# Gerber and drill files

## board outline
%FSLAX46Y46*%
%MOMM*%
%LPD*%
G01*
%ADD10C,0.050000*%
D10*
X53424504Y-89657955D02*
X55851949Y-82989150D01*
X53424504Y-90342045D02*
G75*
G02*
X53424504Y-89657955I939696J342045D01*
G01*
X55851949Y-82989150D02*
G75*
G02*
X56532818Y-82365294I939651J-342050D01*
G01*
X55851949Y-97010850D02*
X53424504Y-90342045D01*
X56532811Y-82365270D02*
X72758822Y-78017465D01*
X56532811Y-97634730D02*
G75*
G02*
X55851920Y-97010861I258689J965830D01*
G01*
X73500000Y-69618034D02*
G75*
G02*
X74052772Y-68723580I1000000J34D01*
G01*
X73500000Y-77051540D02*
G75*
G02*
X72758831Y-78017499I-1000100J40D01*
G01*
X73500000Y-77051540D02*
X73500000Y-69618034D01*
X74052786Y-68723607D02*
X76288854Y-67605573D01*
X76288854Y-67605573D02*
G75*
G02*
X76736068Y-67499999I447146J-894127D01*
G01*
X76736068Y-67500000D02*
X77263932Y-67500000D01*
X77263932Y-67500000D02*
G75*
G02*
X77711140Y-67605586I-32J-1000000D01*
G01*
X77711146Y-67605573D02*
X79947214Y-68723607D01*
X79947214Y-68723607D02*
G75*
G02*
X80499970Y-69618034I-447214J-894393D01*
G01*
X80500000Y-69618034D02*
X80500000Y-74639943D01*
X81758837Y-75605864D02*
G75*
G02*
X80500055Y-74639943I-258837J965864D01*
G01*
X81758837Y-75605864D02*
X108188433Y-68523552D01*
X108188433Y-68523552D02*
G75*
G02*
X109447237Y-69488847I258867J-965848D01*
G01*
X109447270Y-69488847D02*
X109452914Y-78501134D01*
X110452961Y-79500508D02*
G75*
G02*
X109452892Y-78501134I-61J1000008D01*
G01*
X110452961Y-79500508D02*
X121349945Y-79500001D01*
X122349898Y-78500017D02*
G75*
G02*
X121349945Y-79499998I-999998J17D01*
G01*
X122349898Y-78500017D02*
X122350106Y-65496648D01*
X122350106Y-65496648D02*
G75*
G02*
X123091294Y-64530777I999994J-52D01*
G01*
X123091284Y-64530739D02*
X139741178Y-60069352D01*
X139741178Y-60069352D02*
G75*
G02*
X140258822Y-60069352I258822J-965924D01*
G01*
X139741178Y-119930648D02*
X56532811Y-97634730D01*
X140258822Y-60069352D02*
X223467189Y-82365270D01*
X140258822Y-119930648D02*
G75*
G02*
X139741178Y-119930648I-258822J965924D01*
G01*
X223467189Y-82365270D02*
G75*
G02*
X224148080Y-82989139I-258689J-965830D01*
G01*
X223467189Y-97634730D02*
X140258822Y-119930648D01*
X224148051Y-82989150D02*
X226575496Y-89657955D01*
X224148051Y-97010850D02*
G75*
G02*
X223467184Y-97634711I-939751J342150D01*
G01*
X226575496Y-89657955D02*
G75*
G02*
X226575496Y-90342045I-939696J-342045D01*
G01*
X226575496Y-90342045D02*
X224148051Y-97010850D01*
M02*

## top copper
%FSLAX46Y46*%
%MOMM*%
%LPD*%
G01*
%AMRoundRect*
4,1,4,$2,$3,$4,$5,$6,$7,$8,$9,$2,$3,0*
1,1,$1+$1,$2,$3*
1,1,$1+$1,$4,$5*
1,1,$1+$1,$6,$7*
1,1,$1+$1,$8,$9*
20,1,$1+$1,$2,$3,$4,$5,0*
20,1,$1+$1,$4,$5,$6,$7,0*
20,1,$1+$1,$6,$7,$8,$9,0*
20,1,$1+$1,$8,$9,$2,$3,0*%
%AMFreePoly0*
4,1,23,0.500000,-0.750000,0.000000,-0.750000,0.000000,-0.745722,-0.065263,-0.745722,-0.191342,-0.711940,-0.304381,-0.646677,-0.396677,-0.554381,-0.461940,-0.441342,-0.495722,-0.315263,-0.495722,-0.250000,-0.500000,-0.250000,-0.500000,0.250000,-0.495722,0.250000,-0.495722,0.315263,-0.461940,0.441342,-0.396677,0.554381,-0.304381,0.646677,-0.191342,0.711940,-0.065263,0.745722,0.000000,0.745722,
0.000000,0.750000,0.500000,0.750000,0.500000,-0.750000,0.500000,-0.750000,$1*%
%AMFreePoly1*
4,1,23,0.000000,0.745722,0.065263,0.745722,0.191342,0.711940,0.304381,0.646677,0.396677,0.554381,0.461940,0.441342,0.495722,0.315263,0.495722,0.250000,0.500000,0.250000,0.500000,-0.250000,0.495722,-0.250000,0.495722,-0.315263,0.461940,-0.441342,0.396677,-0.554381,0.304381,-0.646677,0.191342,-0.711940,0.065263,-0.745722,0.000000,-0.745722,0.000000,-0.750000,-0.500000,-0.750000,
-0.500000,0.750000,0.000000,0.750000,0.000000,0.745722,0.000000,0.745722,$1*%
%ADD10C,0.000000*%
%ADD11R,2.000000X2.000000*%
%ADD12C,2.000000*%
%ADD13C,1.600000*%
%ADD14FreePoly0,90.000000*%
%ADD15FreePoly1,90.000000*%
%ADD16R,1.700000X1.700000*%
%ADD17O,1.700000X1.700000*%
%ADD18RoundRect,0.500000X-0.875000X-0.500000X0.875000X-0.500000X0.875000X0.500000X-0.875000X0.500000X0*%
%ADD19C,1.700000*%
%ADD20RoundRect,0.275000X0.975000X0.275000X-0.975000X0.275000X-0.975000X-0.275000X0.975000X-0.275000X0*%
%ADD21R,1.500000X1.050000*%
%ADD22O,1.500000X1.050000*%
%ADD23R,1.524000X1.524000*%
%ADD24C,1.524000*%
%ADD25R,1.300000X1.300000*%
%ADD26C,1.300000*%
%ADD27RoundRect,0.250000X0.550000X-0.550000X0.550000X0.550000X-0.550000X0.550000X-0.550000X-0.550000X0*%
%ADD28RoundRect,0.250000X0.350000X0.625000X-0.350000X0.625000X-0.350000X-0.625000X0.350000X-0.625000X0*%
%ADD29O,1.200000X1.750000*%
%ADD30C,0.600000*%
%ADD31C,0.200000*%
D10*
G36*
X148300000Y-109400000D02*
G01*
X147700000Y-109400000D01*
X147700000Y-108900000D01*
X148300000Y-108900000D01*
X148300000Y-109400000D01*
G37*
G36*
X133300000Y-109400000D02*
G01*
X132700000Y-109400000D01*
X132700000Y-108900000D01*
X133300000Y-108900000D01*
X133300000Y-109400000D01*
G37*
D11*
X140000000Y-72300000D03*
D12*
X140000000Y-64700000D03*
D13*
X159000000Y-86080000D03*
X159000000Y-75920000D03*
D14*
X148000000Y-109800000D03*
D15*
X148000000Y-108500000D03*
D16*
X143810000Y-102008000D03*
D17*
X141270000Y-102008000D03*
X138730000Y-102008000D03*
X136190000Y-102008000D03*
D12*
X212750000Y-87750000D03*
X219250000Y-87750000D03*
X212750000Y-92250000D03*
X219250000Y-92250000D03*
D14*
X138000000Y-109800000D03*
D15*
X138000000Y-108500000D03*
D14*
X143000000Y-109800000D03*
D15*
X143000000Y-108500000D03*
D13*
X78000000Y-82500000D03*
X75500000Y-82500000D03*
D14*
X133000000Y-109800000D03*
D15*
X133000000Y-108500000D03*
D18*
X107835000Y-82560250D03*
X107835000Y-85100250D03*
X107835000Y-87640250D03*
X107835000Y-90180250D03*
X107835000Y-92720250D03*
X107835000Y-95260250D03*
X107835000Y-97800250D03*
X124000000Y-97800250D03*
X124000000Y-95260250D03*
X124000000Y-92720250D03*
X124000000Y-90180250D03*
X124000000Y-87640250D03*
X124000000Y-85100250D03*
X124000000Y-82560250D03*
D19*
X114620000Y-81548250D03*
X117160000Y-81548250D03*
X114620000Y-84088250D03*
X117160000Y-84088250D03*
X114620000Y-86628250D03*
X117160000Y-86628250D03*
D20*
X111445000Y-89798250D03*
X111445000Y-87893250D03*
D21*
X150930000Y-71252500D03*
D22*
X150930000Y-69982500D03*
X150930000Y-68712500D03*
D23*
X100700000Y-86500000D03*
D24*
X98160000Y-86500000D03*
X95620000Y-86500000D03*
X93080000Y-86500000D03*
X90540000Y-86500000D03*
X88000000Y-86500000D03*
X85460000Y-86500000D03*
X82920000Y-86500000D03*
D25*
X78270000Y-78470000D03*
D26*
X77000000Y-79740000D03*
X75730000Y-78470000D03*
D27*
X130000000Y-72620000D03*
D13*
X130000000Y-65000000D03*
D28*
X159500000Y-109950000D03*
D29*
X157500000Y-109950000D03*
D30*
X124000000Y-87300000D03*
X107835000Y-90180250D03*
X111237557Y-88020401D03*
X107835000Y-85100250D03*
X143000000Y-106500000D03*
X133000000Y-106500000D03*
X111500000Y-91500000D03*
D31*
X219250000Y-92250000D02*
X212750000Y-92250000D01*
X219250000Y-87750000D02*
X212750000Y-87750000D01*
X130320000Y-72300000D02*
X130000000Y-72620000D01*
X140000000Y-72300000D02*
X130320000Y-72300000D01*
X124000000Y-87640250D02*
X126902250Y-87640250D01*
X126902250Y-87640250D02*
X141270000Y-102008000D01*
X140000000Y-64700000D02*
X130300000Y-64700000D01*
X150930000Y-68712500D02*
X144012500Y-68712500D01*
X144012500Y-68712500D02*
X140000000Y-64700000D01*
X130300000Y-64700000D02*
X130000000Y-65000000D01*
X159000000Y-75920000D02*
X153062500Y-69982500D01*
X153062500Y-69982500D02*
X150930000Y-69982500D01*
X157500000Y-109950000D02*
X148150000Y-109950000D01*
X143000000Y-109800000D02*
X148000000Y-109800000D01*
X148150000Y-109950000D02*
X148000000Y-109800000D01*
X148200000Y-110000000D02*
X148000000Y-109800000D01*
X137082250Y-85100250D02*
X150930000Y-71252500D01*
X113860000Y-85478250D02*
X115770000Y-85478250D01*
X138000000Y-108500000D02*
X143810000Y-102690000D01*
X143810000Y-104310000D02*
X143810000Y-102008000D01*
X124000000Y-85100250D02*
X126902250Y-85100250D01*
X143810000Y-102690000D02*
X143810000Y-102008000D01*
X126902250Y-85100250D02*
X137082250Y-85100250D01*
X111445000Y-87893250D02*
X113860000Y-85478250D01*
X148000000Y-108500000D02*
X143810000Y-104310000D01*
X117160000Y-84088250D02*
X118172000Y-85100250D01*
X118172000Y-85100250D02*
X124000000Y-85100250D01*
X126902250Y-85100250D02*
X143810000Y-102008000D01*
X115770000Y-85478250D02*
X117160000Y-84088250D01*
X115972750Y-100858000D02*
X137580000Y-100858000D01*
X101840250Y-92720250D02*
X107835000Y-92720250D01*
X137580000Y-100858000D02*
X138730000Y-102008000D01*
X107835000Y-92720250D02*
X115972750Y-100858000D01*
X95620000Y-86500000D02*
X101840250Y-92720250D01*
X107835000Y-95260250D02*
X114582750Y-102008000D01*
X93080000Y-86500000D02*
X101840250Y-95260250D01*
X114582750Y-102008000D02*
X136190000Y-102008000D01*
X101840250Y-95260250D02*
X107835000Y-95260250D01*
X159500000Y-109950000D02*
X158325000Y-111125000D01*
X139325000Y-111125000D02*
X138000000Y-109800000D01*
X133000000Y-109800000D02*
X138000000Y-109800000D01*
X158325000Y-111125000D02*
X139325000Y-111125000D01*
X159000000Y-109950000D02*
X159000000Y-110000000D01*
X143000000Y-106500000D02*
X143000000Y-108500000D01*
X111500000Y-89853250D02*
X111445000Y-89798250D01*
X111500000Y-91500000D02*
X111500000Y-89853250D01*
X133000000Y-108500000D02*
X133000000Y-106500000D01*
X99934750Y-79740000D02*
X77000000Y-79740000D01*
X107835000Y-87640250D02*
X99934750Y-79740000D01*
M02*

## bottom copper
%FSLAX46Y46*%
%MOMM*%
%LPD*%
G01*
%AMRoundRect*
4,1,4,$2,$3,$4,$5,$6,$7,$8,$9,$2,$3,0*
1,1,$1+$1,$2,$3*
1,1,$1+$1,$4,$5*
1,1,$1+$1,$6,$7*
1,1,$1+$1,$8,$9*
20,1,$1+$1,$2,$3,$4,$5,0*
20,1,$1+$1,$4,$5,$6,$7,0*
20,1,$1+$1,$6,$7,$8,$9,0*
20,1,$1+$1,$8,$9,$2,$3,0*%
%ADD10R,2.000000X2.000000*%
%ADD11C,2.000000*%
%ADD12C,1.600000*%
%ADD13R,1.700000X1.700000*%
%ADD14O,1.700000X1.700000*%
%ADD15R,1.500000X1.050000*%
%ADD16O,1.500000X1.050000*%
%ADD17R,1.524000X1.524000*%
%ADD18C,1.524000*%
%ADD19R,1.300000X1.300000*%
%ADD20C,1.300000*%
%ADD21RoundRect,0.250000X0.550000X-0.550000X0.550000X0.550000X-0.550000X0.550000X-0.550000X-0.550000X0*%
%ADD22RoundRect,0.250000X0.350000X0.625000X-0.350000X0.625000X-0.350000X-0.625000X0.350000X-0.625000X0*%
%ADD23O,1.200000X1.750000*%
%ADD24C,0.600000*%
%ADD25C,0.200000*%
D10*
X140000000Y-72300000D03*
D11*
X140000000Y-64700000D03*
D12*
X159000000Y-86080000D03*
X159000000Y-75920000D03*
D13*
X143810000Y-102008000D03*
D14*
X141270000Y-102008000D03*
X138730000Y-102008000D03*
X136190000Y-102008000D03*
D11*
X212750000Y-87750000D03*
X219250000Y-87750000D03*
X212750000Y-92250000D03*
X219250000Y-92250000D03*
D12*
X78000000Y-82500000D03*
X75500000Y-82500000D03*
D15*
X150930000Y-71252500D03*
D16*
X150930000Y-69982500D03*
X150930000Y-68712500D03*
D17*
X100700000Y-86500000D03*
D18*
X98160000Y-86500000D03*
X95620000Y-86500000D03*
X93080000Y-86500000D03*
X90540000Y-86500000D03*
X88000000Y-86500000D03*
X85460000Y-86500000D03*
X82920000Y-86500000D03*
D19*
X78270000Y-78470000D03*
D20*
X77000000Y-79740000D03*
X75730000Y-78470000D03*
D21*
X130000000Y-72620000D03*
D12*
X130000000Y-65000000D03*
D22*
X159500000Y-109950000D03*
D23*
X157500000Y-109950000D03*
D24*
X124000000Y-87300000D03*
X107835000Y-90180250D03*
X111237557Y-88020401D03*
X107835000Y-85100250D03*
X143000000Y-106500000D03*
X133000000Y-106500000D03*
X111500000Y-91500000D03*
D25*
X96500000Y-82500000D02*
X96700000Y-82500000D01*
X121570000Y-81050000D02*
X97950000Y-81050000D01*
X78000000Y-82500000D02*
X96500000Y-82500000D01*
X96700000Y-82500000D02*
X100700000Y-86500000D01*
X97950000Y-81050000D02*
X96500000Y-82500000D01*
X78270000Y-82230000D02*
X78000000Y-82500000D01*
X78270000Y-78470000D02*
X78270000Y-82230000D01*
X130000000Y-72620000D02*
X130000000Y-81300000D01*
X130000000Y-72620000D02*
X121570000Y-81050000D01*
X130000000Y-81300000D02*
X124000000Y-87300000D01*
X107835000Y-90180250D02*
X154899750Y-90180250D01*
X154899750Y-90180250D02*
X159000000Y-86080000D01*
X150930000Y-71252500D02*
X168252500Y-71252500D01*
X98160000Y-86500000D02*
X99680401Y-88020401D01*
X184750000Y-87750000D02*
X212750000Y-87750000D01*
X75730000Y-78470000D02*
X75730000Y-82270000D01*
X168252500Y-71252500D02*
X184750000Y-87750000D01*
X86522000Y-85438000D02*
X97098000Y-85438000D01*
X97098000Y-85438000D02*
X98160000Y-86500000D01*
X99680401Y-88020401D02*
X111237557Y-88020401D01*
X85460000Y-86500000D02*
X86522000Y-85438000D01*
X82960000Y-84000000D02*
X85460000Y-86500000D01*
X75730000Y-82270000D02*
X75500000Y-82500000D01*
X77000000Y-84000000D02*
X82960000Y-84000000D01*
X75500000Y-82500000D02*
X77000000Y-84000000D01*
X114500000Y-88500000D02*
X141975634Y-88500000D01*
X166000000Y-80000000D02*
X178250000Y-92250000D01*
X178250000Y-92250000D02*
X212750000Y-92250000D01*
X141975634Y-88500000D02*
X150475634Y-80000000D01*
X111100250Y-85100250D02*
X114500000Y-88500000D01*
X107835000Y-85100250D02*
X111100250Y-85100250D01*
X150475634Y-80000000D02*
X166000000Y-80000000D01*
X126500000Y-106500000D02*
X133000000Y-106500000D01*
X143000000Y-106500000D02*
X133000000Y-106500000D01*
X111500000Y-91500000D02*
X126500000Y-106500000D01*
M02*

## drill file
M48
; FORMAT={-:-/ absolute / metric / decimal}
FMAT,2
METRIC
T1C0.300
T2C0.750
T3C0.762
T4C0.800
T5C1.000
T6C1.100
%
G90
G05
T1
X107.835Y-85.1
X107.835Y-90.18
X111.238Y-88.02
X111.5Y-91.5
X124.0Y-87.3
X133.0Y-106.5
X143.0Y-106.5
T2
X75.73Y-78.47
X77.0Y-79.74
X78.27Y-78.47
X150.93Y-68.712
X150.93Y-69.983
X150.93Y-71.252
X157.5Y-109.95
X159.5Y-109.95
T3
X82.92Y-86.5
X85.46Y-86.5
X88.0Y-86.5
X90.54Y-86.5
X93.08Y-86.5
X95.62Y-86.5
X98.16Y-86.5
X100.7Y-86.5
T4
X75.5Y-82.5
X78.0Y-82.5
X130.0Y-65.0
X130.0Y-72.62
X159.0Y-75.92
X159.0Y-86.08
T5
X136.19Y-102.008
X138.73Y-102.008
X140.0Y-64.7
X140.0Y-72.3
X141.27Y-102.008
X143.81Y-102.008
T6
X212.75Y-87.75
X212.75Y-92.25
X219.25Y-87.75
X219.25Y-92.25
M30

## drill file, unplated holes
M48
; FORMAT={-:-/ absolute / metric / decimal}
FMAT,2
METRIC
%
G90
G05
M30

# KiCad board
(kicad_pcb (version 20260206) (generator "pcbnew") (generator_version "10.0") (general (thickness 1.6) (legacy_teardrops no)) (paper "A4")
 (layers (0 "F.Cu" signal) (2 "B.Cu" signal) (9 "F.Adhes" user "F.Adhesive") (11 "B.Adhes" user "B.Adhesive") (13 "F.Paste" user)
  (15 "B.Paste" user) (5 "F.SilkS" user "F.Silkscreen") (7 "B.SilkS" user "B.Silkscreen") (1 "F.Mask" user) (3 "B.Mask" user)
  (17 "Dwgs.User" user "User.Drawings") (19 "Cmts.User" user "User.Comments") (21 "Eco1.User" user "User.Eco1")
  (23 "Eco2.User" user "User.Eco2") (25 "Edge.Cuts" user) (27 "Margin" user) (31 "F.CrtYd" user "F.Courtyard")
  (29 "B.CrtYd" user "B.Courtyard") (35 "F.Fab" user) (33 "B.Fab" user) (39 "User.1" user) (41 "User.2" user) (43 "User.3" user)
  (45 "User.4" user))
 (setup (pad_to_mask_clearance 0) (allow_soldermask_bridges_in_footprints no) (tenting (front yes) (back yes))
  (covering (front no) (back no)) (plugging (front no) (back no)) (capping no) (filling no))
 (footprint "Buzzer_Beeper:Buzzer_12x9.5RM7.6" (layer "F.Cu") (at 140 72.3 90)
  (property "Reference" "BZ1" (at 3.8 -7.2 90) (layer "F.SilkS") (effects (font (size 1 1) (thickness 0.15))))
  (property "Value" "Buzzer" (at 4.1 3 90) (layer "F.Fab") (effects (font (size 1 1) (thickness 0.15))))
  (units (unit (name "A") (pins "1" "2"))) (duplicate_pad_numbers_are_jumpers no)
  (pad "1" thru_hole rect (at 0 0 90) (size 2 2) (drill 1) (layers "*.Cu" "*.Mask") (remove_unused_layers no) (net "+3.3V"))
  (pad "2" thru_hole circle (at 7.6 0 90) (size 2 2) (drill 1) (layers "*.Cu" "*.Mask") (remove_unused_layers no) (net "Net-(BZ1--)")))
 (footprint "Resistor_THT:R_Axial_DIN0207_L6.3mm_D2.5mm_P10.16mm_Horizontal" (layer "F.Cu") (at 159 86.08 90)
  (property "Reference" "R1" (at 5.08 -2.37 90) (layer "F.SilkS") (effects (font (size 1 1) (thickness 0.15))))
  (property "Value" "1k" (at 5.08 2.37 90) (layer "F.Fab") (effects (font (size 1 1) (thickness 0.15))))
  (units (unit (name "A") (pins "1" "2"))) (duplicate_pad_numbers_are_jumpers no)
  (pad "1" thru_hole circle (at 0 0 90) (size 1.6 1.6) (drill 0.8) (layers "*.Cu" "*.Mask") (remove_unused_layers no)
   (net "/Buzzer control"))
  (pad "2" thru_hole circle (at 10.16 0 90) (size 1.6 1.6) (drill 0.8) (layers "*.Cu" "*.Mask") (remove_unused_layers no) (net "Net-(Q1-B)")))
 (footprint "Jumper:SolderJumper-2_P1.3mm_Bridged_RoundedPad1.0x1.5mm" (layer "F.Cu") (at 148 109.15 90)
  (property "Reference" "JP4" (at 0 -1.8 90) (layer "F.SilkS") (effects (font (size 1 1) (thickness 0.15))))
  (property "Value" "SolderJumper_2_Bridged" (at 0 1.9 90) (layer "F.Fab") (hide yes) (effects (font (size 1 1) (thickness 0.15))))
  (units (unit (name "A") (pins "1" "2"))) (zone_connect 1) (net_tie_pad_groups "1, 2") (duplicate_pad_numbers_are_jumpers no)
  (fp_poly (pts (xy 0.25 -0.3) (xy -0.25 -0.3) (xy -0.25 0.3) (xy 0.25 0.3)) (stroke (width 0) (type solid)) (fill yes) (layer "F.Cu"))
  (pad "1" smd custom (at -0.65 0 90) (size 1 0.5) (layers "F.Cu" "F.Mask") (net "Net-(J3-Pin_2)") (zone_connect 2)
   (thermal_bridge_angle 45) (options (clearance outline) (anchor rect)) (primitives))
  (pad "2" smd custom (at 0.65 0 90) (size 1 0.5) (layers "F.Cu" "F.Mask") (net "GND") (zone_connect 2) (thermal_bridge_angle 45)
   (options (clearance outline) (anchor rect)) (primitives)))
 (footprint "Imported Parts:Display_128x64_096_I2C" (layer "F.Cu") (at 140 102.008 180)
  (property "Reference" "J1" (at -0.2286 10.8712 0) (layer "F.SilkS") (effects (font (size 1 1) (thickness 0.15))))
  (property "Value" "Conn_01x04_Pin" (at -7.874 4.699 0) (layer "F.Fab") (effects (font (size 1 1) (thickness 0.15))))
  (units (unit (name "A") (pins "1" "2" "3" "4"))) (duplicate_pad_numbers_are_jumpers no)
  (pad "1" thru_hole rect (at -3.81 0 270) (size 1.7 1.7) (drill 1) (layers "*.Cu" "*.Mask") (remove_unused_layers no) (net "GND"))
  (pad "2" thru_hole oval (at -1.27 0 270) (size 1.7 1.7) (drill 1) (layers "*.Cu" "*.Mask") (remove_unused_layers no) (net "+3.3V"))
  (pad "3" thru_hole oval (at 1.27 0 270) (size 1.7 1.7) (drill 1) (layers "*.Cu" "*.Mask") (remove_unused_layers no) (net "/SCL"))
  (pad "4" thru_hole oval (at 3.81 0 270) (size 1.7 1.7) (drill 1) (layers "*.Cu" "*.Mask") (remove_unused_layers no) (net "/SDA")))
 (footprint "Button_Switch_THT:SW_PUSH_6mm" (layer "F.Cu") (at 212.75 87.75)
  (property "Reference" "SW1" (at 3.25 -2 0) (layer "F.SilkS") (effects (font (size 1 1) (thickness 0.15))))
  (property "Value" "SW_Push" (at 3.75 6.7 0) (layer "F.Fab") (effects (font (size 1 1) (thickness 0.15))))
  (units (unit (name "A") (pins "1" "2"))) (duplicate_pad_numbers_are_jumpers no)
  (pad "1" thru_hole circle (at 0 0 90) (size 2 2) (drill 1.1) (layers "*.Cu" "*.Mask") (remove_unused_layers no) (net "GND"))
  (pad "1" thru_hole circle (at 6.5 0 90) (size 2 2) (drill 1.1) (layers "*.Cu" "*.Mask") (remove_unused_layers no) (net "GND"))
  (pad "2" thru_hole circle (at 0 4.5 90) (size 2 2) (drill 1.1) (layers "*.Cu" "*.Mask") (remove_unused_layers no) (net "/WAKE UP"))
  (pad "2" thru_hole circle (at 6.5 4.5 90) (size 2 2) (drill 1.1) (layers "*.Cu" "*.Mask") (remove_unused_layers no) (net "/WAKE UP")))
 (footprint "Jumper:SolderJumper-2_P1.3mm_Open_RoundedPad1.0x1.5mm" (layer "F.Cu") (at 138 109.15 90)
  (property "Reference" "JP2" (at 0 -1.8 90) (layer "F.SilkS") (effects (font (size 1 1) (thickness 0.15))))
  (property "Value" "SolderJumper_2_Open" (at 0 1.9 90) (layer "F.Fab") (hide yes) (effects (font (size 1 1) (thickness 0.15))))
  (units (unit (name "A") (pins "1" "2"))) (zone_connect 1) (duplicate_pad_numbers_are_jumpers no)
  (pad "1" smd custom (at -0.65 0 90) (size 1 0.5) (layers "F.Cu" "F.Mask") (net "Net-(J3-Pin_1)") (zone_connect 2)
   (thermal_bridge_angle 45) (options (clearance outline) (anchor rect)) (primitives))
  (pad "2" smd custom (at 0.65 0 90) (size 1 0.5) (layers "F.Cu" "F.Mask") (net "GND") (zone_connect 2) (thermal_bridge_angle 45)
   (options (clearance outline) (anchor rect)) (primitives)))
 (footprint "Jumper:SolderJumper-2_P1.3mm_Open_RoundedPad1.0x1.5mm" (layer "F.Cu") (at 143 109.15 90)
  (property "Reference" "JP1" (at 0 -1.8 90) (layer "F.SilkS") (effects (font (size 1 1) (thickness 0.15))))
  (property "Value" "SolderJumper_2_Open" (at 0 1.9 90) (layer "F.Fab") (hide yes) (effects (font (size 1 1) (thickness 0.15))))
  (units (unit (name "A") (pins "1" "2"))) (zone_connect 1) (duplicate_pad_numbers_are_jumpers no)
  (pad "1" smd custom (at -0.65 0 90) (size 1 0.5) (layers "F.Cu" "F.Mask") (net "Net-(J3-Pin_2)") (zone_connect 2)
   (thermal_bridge_angle 45) (options (clearance outline) (anchor rect)) (primitives))
  (pad "2" smd custom (at 0.65 0 90) (size 1 0.5) (layers "F.Cu" "F.Mask") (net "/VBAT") (zone_connect 2) (thermal_bridge_angle 45)
   (options (clearance outline) (anchor rect)) (primitives)))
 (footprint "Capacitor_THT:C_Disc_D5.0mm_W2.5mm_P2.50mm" (layer "F.Cu") (at 78 82.5 180)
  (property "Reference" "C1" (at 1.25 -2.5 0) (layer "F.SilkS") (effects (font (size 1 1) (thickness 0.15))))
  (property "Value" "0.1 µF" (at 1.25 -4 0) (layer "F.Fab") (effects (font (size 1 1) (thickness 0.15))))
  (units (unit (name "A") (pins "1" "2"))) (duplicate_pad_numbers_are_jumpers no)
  (pad "1" thru_hole circle (at 0 0 180) (size 1.6 1.6) (drill 0.8) (layers "*.Cu" "*.Mask") (remove_unused_layers no) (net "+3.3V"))
  (pad "2" thru_hole circle (at 2.5 0 180) (size 1.6 1.6) (drill 0.8) (layers "*.Cu" "*.Mask") (remove_unused_layers no) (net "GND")))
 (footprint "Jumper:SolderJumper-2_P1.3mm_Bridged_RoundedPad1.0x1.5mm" (layer "F.Cu") (at 133 109.15 90)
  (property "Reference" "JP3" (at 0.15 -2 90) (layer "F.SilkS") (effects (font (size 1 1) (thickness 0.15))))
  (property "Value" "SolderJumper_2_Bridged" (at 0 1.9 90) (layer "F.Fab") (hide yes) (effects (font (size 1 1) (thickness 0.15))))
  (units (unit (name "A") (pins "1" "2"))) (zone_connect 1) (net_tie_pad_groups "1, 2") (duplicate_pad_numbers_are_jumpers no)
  (fp_poly (pts (xy 0.25 -0.3) (xy -0.25 -0.3) (xy -0.25 0.3) (xy 0.25 0.3)) (stroke (width 0) (type solid)) (fill yes) (layer "F.Cu"))
  (pad "1" smd custom (at -0.65 0 90) (size 1 0.5) (layers "F.Cu" "F.Mask") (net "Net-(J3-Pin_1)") (zone_connect 2)
   (thermal_bridge_angle 45) (options (clearance outline) (anchor rect)) (primitives))
  (pad "2" smd custom (at 0.65 0 90) (size 1 0.5) (layers "F.Cu" "F.Mask") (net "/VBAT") (zone_connect 2) (thermal_bridge_angle 45)
   (options (clearance outline) (anchor rect)) (primitives)))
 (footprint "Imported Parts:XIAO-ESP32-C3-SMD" (layer "F.Cu") (at 107 100.68025)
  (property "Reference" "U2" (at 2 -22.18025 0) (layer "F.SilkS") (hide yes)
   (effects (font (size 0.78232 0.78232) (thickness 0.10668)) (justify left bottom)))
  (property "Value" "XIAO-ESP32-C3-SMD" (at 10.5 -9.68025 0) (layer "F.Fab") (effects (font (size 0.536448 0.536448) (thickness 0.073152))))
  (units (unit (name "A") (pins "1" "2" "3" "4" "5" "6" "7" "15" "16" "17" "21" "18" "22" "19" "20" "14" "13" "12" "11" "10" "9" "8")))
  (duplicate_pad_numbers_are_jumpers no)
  (pad "1" smd roundrect (at 0.835 -18.12) (size 2.75 2) (layers "F.Cu" "F.Mask" "F.Paste") (roundrect_rratio 0.25)
   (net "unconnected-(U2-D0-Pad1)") (solder_mask_margin 0.0508) (thermal_bridge_angle 45))
  (pad "2" smd roundrect (at 0.835 -15.58) (size 2.75 2) (layers "F.Cu" "F.Mask" "F.Paste") (roundrect_rratio 0.25) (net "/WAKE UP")
   (solder_mask_margin 0.0508) (thermal_bridge_angle 45))
  (pad "3" smd roundrect (at 0.835 -13.04) (size 2.75 2) (layers "F.Cu" "F.Mask" "F.Paste") (roundrect_rratio 0.25) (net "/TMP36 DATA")
   (solder_mask_margin 0.0508) (thermal_bridge_angle 45))
  (pad "4" smd roundrect (at 0.835 -10.5) (size 2.75 2) (layers "F.Cu" "F.Mask" "F.Paste") (roundrect_rratio 0.25) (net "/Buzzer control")
   (solder_mask_margin 0.0508) (thermal_bridge_angle 45))
  (pad "5" smd roundrect (at 0.835 -7.96) (size 2.75 2) (layers "F.Cu" "F.Mask" "F.Paste") (roundrect_rratio 0.25) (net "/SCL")
   (solder_mask_margin 0.0508) (thermal_bridge_angle 45))
  (pad "6" smd roundrect (at 0.835 -5.42) (size 2.75 2) (layers "F.Cu" "F.Mask" "F.Paste") (roundrect_rratio 0.25) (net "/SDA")
   (solder_mask_margin 0.0508) (thermal_bridge_angle 45))
  (pad "7" smd roundrect (at 0.835 -2.88) (size 2.75 2) (layers "F.Cu" "F.Mask" "F.Paste") (roundrect_rratio 0.25)
   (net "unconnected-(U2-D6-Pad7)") (solder_mask_margin 0.0508) (thermal_bridge_angle 45))
  (pad "8" smd roundrect (at 17 -2.88) (size 2.75 2) (layers "F.Cu" "F.Mask" "F.Paste") (roundrect_rratio 0.25)
   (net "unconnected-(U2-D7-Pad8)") (solder_mask_margin 0.0508) (thermal_bridge_angle 45))
  (pad "9" smd roundrect (at 17 -5.42) (size 2.75 2) (layers "F.Cu" "F.Mask" "F.Paste") (roundrect_rratio 0.25)
   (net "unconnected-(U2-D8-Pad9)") (solder_mask_margin 0.0508) (thermal_bridge_angle 45))
  (pad "10" smd roundrect (at 17 -7.96) (size 2.75 2) (layers "F.Cu" "F.Mask" "F.Paste") (roundrect_rratio 0.25)
   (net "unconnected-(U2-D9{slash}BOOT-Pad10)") (solder_mask_margin 0.0508) (thermal_bridge_angle 45))
  (pad "11" smd roundrect (at 17 -10.5) (size 2.75 2) (layers "F.Cu" "F.Mask" "F.Paste") (roundrect_rratio 0.25)
   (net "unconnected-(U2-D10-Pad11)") (solder_mask_margin 0.0508) (thermal_bridge_angle 45))
  (pad "12" smd roundrect (at 17 -13.04) (size 2.75 2) (layers "F.Cu" "F.Mask" "F.Paste") (roundrect_rratio 0.25) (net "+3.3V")
   (solder_mask_margin 0.0508) (thermal_bridge_angle 45))
  (pad "13" smd roundrect (at 17 -15.58) (size 2.75 2) (layers "F.Cu" "F.Mask" "F.Paste") (roundrect_rratio 0.25) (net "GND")
   (solder_mask_margin 0.0508) (thermal_bridge_angle 45))
  (pad "14" smd roundrect (at 17 -18.12) (size 2.75 2) (layers "F.Cu" "F.Mask" "F.Paste") (roundrect_rratio 0.25) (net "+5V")
   (solder_mask_margin 0.0508) (thermal_bridge_angle 45))
  (pad "15" smd circle (at 7.62 -19.132) (size 1.7 1.7) (layers "F.Cu" "F.Mask" "F.Paste") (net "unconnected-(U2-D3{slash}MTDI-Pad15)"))
  (pad "16" smd circle (at 10.16 -19.132) (size 1.7 1.7) (layers "F.Cu" "F.Mask" "F.Paste") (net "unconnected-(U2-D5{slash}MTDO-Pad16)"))
  (pad "17" smd circle (at 7.62 -16.592) (size 1.7 1.7) (layers "F.Cu" "F.Mask" "F.Paste") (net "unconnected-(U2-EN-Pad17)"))
  (pad "18" smd circle (at 10.16 -16.592) (size 1.7 1.7) (layers "F.Cu" "F.Mask" "F.Paste") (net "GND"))
  (pad "19" smd circle (at 7.62 -14.052) (size 1.7 1.7) (layers "F.Cu" "F.Mask" "F.Paste") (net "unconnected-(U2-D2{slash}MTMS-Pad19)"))
  (pad "20" smd circle (at 10.16 -14.052) (size 1.7 1.7) (layers "F.Cu" "F.Mask" "F.Paste") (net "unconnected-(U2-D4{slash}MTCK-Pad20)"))
  (pad "21" smd roundrect (at 4.445 -10.882 180) (size 2.5 1.1) (layers "F.Cu" "F.Mask" "F.Paste") (roundrect_rratio 0.25) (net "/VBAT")
   (thermal_bridge_angle 45))
  (pad "22" smd roundrect (at 4.445 -12.787 180) (size 2.5 1.1) (layers "F.Cu" "F.Mask" "F.Paste") (roundrect_rratio 0.25) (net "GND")
   (thermal_bridge_angle 45)))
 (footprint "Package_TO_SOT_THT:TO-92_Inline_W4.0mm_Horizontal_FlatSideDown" (layer "F.Cu") (at 150.93 71.2525 90)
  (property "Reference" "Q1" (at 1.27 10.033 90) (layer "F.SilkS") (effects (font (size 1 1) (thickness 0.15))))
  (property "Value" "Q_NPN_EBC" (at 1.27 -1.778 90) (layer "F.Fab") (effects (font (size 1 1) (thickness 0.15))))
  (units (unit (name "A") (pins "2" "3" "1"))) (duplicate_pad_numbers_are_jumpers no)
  (pad "1" thru_hole rect (at 0 0 90) (size 1.05 1.5) (drill 0.75) (layers "*.Cu" "*.Mask") (remove_unused_layers no) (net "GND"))
  (pad "2" thru_hole oval (at 1.27 0 90) (size 1.05 1.5) (drill 0.75) (layers "*.Cu" "*.Mask") (remove_unused_layers no) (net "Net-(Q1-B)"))
  (pad "3" thru_hole oval (at 2.54 0 90) (size 1.05 1.5) (drill 0.75) (layers "*.Cu" "*.Mask") (remove_unused_layers no) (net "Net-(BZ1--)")))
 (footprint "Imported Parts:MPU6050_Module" (layer "F.Cu") (at 100.7 86.5 -90)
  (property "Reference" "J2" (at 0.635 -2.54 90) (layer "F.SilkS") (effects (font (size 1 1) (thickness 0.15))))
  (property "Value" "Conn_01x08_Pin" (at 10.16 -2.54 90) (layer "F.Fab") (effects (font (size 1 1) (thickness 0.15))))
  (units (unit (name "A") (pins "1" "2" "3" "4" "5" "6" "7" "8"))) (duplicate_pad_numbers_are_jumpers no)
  (pad "1" thru_hole rect (at 0 0 270) (size 1.524 1.524) (drill 0.762) (layers "*.Cu" "*.Mask") (remove_unused_layers no) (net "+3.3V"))
  (pad "2" thru_hole circle (at 0 2.54 270) (size 1.524 1.524) (drill 0.762) (layers "*.Cu" "*.Mask") (remove_unused_layers no) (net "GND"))
  (pad "3" thru_hole circle (at 0 5.08 270) (size 1.524 1.524) (drill 0.762) (layers "*.Cu" "*.Mask") (remove_unused_layers no) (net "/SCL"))
  (pad "4" thru_hole circle (at 0 7.62 270) (size 1.524 1.524) (drill 0.762) (layers "*.Cu" "*.Mask") (remove_unused_layers no) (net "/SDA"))
  (pad "5" thru_hole circle (at 0 10.16 270) (size 1.524 1.524) (drill 0.762) (layers "*.Cu" "*.Mask") (remove_unused_layers no)
   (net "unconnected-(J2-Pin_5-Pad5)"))
  (pad "6" thru_hole circle (at 0 12.7 270) (size 1.524 1.524) (drill 0.762) (layers "*.Cu" "*.Mask") (remove_unused_layers no)
   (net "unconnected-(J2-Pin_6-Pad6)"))
  (pad "7" thru_hole circle (at 0 15.24 270) (size 1.524 1.524) (drill 0.762) (layers "*.Cu" "*.Mask") (remove_unused_layers no) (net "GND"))
  (pad "8" thru_hole circle (at 0 17.78 270) (size 1.524 1.524) (drill 0.762) (layers "*.Cu" "*.Mask") (remove_unused_layers no)
   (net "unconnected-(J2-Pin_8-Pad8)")))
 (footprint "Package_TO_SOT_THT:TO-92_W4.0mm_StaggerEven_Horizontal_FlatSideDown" (layer "F.Cu") (at 78.27 78.47 180)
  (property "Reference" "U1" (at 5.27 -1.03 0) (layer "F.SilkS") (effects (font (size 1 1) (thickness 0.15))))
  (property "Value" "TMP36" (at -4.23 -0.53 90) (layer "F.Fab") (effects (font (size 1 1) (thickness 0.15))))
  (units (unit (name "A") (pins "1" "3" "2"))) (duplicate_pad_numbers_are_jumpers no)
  (pad "1" thru_hole rect (at 0 0 270) (size 1.3 1.3) (drill 0.75) (layers "*.Cu" "*.Mask") (remove_unused_layers no) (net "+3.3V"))
  (pad "2" thru_hole circle (at 1.27 -1.27 270) (size 1.3 1.3) (drill 0.75) (layers "*.Cu" "*.Mask") (remove_unused_layers no)
   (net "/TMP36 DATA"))
  (pad "3" thru_hole circle (at 2.54 0 270) (size 1.3 1.3) (drill 0.75) (layers "*.Cu" "*.Mask") (remove_unused_layers no) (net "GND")))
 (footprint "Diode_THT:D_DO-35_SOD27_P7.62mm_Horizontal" (layer "F.Cu") (at 130 72.62 90)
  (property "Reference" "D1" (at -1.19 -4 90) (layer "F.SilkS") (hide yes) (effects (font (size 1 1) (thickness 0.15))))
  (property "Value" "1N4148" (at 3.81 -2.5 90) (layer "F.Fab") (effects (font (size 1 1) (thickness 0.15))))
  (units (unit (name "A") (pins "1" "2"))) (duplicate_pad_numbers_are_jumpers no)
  (pad "1" thru_hole roundrect (at 0 0 90) (size 1.6 1.6) (drill 0.8) (layers "*.Cu" "*.Mask") (remove_unused_layers no)
   (roundrect_rratio 0.15625) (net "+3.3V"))
  (pad "2" thru_hole circle (at 7.62 0 90) (size 1.6 1.6) (drill 0.8) (layers "*.Cu" "*.Mask") (remove_unused_layers no) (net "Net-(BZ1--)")))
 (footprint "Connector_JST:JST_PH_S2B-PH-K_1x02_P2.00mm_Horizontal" (layer "F.Cu") (at 159.5 109.95 180)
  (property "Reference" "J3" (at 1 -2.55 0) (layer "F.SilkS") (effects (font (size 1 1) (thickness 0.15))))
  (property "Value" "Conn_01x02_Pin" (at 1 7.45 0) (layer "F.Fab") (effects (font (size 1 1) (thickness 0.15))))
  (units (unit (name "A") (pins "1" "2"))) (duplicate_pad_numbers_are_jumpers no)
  (pad "1" thru_hole roundrect (at 0 0 180) (size 1.2 1.75) (drill 0.75) (layers "*.Cu" "*.Mask") (remove_unused_layers no)
   (roundrect_rratio 0.208333) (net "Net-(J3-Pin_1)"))
  (pad "2" thru_hole oval (at 2 0 180) (size 1.2 1.75) (drill 0.75) (layers "*.Cu" "*.Mask") (remove_unused_layers no)
   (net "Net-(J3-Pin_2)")))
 (gr_line (start 53.424504 89.657955) (end 55.851949 82.98915) (stroke (width 0.05) (type default)) (layer "Edge.Cuts"))
 (gr_arc (start 53.424504 90.342045) (mid 53.364188 90) (end 53.424504 89.657955) (stroke (width 0.05) (type default)) (layer "Edge.Cuts"))
 (gr_arc (start 55.851949 82.98915) (mid 56.116051 82.59391) (end 56.532811 82.36527) (stroke (width 0.05) (type default))
  (layer "Edge.Cuts"))
 (gr_line (start 55.851949 97.01085) (end 53.424504 90.342045) (stroke (width 0.05) (type default)) (layer "Edge.Cuts"))
 (gr_line (start 56.532811 82.36527) (end 72.758822 78.017465) (stroke (width 0.05) (type default)) (layer "Edge.Cuts"))
 (gr_arc (start 56.532811 97.63473) (mid 56.116039 97.406099) (end 55.851949 97.01085) (stroke (width 0.05) (type default))
  (layer "Edge.Cuts"))
 (gr_arc (start 73.5 69.618034) (mid 73.649349 69.092303) (end 74.052786 68.723607) (stroke (width 0.05) (type default)) (layer "Edge.Cuts"))
 (gr_arc (start 73.5 77.05154) (mid 73.293339 77.66028) (end 72.758822 78.017465) (stroke (width 0.05) (type default)) (layer "Edge.Cuts"))
 (gr_line (start 73.5 77.05154) (end 73.5 69.618034) (stroke (width 0.05) (type default)) (layer "Edge.Cuts"))
 (gr_line (start 74.052786 68.723607) (end 76.288854 67.605573) (stroke (width 0.05) (type default)) (layer "Edge.Cuts"))
 (gr_arc (start 76.288854 67.605573) (mid 76.506314 67.526744) (end 76.736068 67.5) (stroke (width 0.05) (type default)) (layer "Edge.Cuts"))
 (gr_line (start 76.736068 67.5) (end 77.263932 67.5) (stroke (width 0.05) (type default)) (layer "Edge.Cuts"))
 (gr_arc (start 77.263932 67.5) (mid 77.493685 67.526751) (end 77.711146 67.605573) (stroke (width 0.05) (type default)) (layer "Edge.Cuts"))
 (gr_line (start 77.711146 67.605573) (end 79.947214 68.723607) (stroke (width 0.05) (type default)) (layer "Edge.Cuts"))
 (gr_arc (start 79.947214 68.723607) (mid 80.350651 69.092303) (end 80.5 69.618034) (stroke (width 0.05) (type default)) (layer "Edge.Cuts"))
 (gr_line (start 80.5 69.618034) (end 80.5 74.639943) (stroke (width 0.05) (type default)) (layer "Edge.Cuts"))
 (gr_arc (start 81.758837 75.605864) (mid 80.891233 75.433302) (end 80.5 74.639943) (stroke (width 0.05) (type default)) (layer "Edge.Cuts"))
 (gr_line (start 81.758837 75.605864) (end 108.188433 68.523552) (stroke (width 0.05) (type default)) (layer "Edge.Cuts"))
 (gr_arc (start 108.188433 68.523552) (mid 109.055807 68.695909) (end 109.44727 69.488847) (stroke (width 0.05) (type default))
  (layer "Edge.Cuts"))
 (gr_line (start 109.44727 69.488847) (end 109.452914 78.501134) (stroke (width 0.05) (type default)) (layer "Edge.Cuts"))
 (gr_arc (start 110.452961 79.500508) (mid 109.746033 79.207858) (end 109.452914 78.501134) (stroke (width 0.05) (type default))
  (layer "Edge.Cuts"))
 (gr_line (start 110.452961 79.500508) (end 121.349945 79.500001) (stroke (width 0.05) (type default)) (layer "Edge.Cuts"))
 (gr_arc (start 122.349898 78.500017) (mid 122.057016 79.207097) (end 121.349945 79.500001) (stroke (width 0.05) (type default))
  (layer "Edge.Cuts"))
 (gr_line (start 122.349898 78.500017) (end 122.350106 65.496648) (stroke (width 0.05) (type default)) (layer "Edge.Cuts"))
 (gr_arc (start 122.350106 65.496648) (mid 122.556757 64.887897) (end 123.091284 64.530739) (stroke (width 0.05) (type default))
  (layer "Edge.Cuts"))
 (gr_line (start 123.091284 64.530739) (end 139.741178 60.069352) (stroke (width 0.05) (type default)) (layer "Edge.Cuts"))
 (gr_arc (start 139.741178 60.069352) (mid 140 60.035277) (end 140.258822 60.069352) (stroke (width 0.05) (type default))
  (layer "Edge.Cuts"))
 (gr_line (start 139.741178 119.930648) (end 56.532811 97.63473) (stroke (width 0.05) (type default)) (layer "Edge.Cuts"))
 (gr_line (start 140.258822 60.069352) (end 223.467189 82.36527) (stroke (width 0.05) (type default)) (layer "Edge.Cuts"))
 (gr_arc (start 140.258822 119.930648) (mid 140 119.964723) (end 139.741178 119.930648) (stroke (width 0.05) (type default))
  (layer "Edge.Cuts"))
 (gr_arc (start 223.467189 82.36527) (mid 223.883961 82.593901) (end 224.148051 82.98915) (stroke (width 0.05) (type default))
  (layer "Edge.Cuts"))
 (gr_line (start 223.467189 97.63473) (end 140.258822 119.930648) (stroke (width 0.05) (type default)) (layer "Edge.Cuts"))
 (gr_line (start 224.148051 82.98915) (end 226.575496 89.657955) (stroke (width 0.05) (type default)) (layer "Edge.Cuts"))
 (gr_arc (start 224.148051 97.01085) (mid 223.883944 97.40608) (end 223.467189 97.63473) (stroke (width 0.05) (type default))
  (layer "Edge.Cuts"))
 (gr_arc (start 226.575496 89.657955) (mid 226.635812 90) (end 226.575496 90.342045) (stroke (width 0.05) (type default))
  (layer "Edge.Cuts"))
 (gr_line (start 226.575496 90.342045) (end 224.148051 97.01085) (stroke (width 0.05) (type default)) (layer "Edge.Cuts"))
 (segment (start 130.32 72.3) (end 130 72.62) (width 0.2) (layer "F.Cu") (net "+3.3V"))
 (segment (start 140 72.3) (end 130.32 72.3) (width 0.2) (layer "F.Cu") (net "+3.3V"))
 (segment (start 124 87.64025) (end 126.90225 87.64025) (width 0.2) (layer "F.Cu") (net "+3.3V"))
 (segment (start 126.90225 87.64025) (end 141.27 102.008) (width 0.2) (layer "F.Cu") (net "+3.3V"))
 (via (at 124 87.3) (size 0.6) (drill 0.3) (layers "F.Cu" "B.Cu") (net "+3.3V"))
 (segment (start 96.5 82.5) (end 96.7 82.5) (width 0.2) (layer "B.Cu") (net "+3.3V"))
 (segment (start 121.57 81.05) (end 97.95 81.05) (width 0.2) (layer "B.Cu") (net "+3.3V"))
 (segment (start 78 82.5) (end 96.5 82.5) (width 0.2) (layer "B.Cu") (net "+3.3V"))
 (segment (start 96.7 82.5) (end 100.7 86.5) (width 0.2) (layer "B.Cu") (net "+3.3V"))
 (segment (start 97.95 81.05) (end 96.5 82.5) (width 0.2) (layer "B.Cu") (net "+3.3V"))
 (segment (start 78.27 82.23) (end 78 82.5) (width 0.2) (layer "B.Cu") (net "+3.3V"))
 (segment (start 78.27 78.47) (end 78.27 82.23) (width 0.2) (layer "B.Cu") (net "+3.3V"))
 (segment (start 130 72.62) (end 130 81.3) (width 0.2) (layer "B.Cu") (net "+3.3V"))
 (segment (start 130 72.62) (end 121.57 81.05) (width 0.2) (layer "B.Cu") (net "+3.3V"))
 (segment (start 130 81.3) (end 124 87.3) (width 0.2) (layer "B.Cu") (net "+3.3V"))
 (segment (start 140 64.7) (end 130.3 64.7) (width 0.2) (layer "F.Cu") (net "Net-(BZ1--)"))
 (segment (start 150.93 68.7125) (end 144.0125 68.7125) (width 0.2) (layer "F.Cu") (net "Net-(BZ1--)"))
 (segment (start 144.0125 68.7125) (end 140 64.7) (width 0.2) (layer "F.Cu") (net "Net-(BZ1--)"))
 (segment (start 130.3 64.7) (end 130 65) (width 0.2) (layer "F.Cu") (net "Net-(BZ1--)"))
 (via (at 107.835 90.18025) (size 0.6) (drill 0.3) (layers "F.Cu" "B.Cu") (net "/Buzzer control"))
 (segment (start 107.835 90.18025) (end 154.89975 90.18025) (width 0.2) (layer "B.Cu") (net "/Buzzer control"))
 (segment (start 154.89975 90.18025) (end 159 86.08) (width 0.2) (layer "B.Cu") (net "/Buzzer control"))
 (segment (start 159 75.92) (end 153.0625 69.9825) (width 0.2) (layer "F.Cu") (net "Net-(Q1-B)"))
 (segment (start 153.0625 69.9825) (end 150.93 69.9825) (width 0.2) (layer "F.Cu") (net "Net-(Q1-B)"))
 (segment (start 157.5 109.95) (end 148.15 109.95) (width 0.2) (layer "F.Cu") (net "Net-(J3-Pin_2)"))
 (segment (start 143 109.8) (end 148 109.8) (width 0.2) (layer "F.Cu") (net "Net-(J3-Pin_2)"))
 (segment (start 148.15 109.95) (end 148 109.8) (width 0.2) (layer "F.Cu") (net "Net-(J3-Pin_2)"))
 (segment (start 148.2 110) (end 148 109.8) (width 0.2) (layer "F.Cu") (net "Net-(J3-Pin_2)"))
 (segment (start 137.08225 85.10025) (end 150.93 71.2525) (width 0.2) (layer "F.Cu") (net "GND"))
 (segment (start 219.25 87.75) (end 212.75 87.75) (width 0.2) (layer "F.Cu") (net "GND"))
 (segment (start 113.86 85.47825) (end 115.77 85.47825) (width 0.2) (layer "F.Cu") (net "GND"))
 (segment (start 138 108.5) (end 143.81 102.69) (width 0.2) (layer "F.Cu") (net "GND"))
 (segment (start 143.81 104.31) (end 143.81 102.008) (width 0.2) (layer "F.Cu") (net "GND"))
 (segment (start 124 85.10025) (end 126.90225 85.10025) (width 0.2) (layer "F.Cu") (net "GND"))
 (segment (start 143.81 102.69) (end 143.81 102.008) (width 0.2) (layer "F.Cu") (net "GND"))
 (segment (start 126.90225 85.10025) (end 137.08225 85.10025) (width 0.2) (layer "F.Cu") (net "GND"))
 (segment (start 111.445 87.89325) (end 113.86 85.47825) (width 0.2) (layer "F.Cu") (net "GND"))
 (segment (start 148 108.5) (end 143.81 104.31) (width 0.2) (layer "F.Cu") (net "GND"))
 (segment (start 117.16 84.08825) (end 118.172 85.10025) (width 0.2) (layer "F.Cu") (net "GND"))
 (segment (start 118.172 85.10025) (end 124 85.10025) (width 0.2) (layer "F.Cu") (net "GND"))
 (segment (start 126.90225 85.10025) (end 143.81 102.008) (width 0.2) (layer "F.Cu") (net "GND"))
 (segment (start 115.77 85.47825) (end 117.16 84.08825) (width 0.2) (layer "F.Cu") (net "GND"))
 (via (at 111.237557 88.020401) (size 0.6) (drill 0.3) (layers "F.Cu" "B.Cu") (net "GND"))
 (segment (start 150.93 71.2525) (end 168.2525 71.2525) (width 0.2) (layer "B.Cu") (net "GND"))
 (segment (start 98.16 86.5) (end 99.680401 88.020401) (width 0.2) (layer "B.Cu") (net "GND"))
 (segment (start 184.75 87.75) (end 212.75 87.75) (width 0.2) (layer "B.Cu") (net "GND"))
 (segment (start 75.73 78.47) (end 75.73 82.27) (width 0.2) (layer "B.Cu") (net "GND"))
 (segment (start 168.2525 71.2525) (end 184.75 87.75) (width 0.2) (layer "B.Cu") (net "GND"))
 (segment (start 86.522 85.438) (end 97.098 85.438) (width 0.2) (layer "B.Cu") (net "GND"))
 (segment (start 97.098 85.438) (end 98.16 86.5) (width 0.2) (layer "B.Cu") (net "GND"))
 (segment (start 99.680401 88.020401) (end 111.237557 88.020401) (width 0.2) (layer "B.Cu") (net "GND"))
 (segment (start 85.46 86.5) (end 86.522 85.438) (width 0.2) (layer "B.Cu") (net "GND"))
 (segment (start 82.96 84) (end 85.46 86.5) (width 0.2) (layer "B.Cu") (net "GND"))
 (segment (start 75.73 82.27) (end 75.5 82.5) (width 0.2) (layer "B.Cu") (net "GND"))
 (segment (start 77 84) (end 82.96 84) (width 0.2) (layer "B.Cu") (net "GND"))
 (segment (start 75.5 82.5) (end 77 84) (width 0.2) (layer "B.Cu") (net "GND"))
 (segment (start 115.97275 100.858) (end 137.58 100.858) (width 0.2) (layer "F.Cu") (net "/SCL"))
 (segment (start 101.84025 92.72025) (end 107.835 92.72025) (width 0.2) (layer "F.Cu") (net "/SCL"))
 (segment (start 137.58 100.858) (end 138.73 102.008) (width 0.2) (layer "F.Cu") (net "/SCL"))
 (segment (start 107.835 92.72025) (end 115.97275 100.858) (width 0.2) (layer "F.Cu") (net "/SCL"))
 (segment (start 95.62 86.5) (end 101.84025 92.72025) (width 0.2) (layer "F.Cu") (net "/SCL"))
 (segment (start 107.835 95.26025) (end 114.58275 102.008) (width 0.2) (layer "F.Cu") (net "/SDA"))
 (segment (start 93.08 86.5) (end 101.84025 95.26025) (width 0.2) (layer "F.Cu") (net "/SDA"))
 (segment (start 114.58275 102.008) (end 136.19 102.008) (width 0.2) (layer "F.Cu") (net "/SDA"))
 (segment (start 101.84025 95.26025) (end 107.835 95.26025) (width 0.2) (layer "F.Cu") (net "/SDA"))
 (segment (start 219.25 92.25) (end 212.75 92.25) (width 0.2) (layer "F.Cu") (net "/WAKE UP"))
 (via (at 107.835 85.10025) (size 0.6) (drill 0.3) (layers "F.Cu" "B.Cu") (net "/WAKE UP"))
 (segment (start 114.5 88.5) (end 141.975634 88.5) (width 0.2) (layer "B.Cu") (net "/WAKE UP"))
 (segment (start 166 80) (end 178.25 92.25) (width 0.2) (layer "B.Cu") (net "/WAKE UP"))
 (segment (start 178.25 92.25) (end 212.75 92.25) (width 0.2) (layer "B.Cu") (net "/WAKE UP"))
 (segment (start 141.975634 88.5) (end 150.475634 80) (width 0.2) (layer "B.Cu") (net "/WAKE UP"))
 (segment (start 111.10025 85.10025) (end 114.5 88.5) (width 0.2) (layer "B.Cu") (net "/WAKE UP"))
 (segment (start 107.835 85.10025) (end 111.10025 85.10025) (width 0.2) (layer "B.Cu") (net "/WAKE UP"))
 (segment (start 150.475634 80) (end 166 80) (width 0.2) (layer "B.Cu") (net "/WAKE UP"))
 (segment (start 159.5 109.95) (end 158.325 111.125) (width 0.2) (layer "F.Cu") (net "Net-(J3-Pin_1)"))
 (segment (start 139.325 111.125) (end 138 109.8) (width 0.2) (layer "F.Cu") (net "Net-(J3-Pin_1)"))
 (segment (start 133 109.8) (end 138 109.8) (width 0.2) (layer "F.Cu") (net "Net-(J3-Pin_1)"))
 (segment (start 158.325 111.125) (end 139.325 111.125) (width 0.2) (layer "F.Cu") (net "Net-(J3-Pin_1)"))
 (segment (start 159 109.95) (end 159 110) (width 0.2) (layer "F.Cu") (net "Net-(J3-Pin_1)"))
 (segment (start 143 106.5) (end 143 108.5) (width 0.2) (layer "F.Cu") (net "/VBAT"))
 (segment (start 111.5 89.85325) (end 111.445 89.79825) (width 0.2) (layer "F.Cu") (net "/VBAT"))
 (segment (start 111.5 91.5) (end 111.5 89.85325) (width 0.2) (layer "F.Cu") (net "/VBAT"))
 (segment (start 133 108.5) (end 133 106.5) (width 0.2) (layer "F.Cu") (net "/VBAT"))
 (via (at 143 106.5) (size 0.6) (drill 0.3) (layers "F.Cu" "B.Cu") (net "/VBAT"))
 (via (at 133 106.5) (size 0.6) (drill 0.3) (layers "F.Cu" "B.Cu") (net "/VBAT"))
 (via (at 111.5 91.5) (size 0.6) (drill 0.3) (layers "F.Cu" "B.Cu") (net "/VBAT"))
 (segment (start 126.5 106.5) (end 133 106.5) (width 0.2) (layer "B.Cu") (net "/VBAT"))
 (segment (start 143 106.5) (end 133 106.5) (width 0.2) (layer "B.Cu") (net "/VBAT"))
 (segment (start 111.5 91.5) (end 126.5 106.5) (width 0.2) (layer "B.Cu") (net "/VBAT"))
 (segment (start 99.93475 79.74) (end 77 79.74) (width 0.2) (layer "F.Cu") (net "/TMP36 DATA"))
 (segment (start 107.835 87.64025) (end 99.93475 79.74) (width 0.2) (layer "F.Cu") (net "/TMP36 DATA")))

